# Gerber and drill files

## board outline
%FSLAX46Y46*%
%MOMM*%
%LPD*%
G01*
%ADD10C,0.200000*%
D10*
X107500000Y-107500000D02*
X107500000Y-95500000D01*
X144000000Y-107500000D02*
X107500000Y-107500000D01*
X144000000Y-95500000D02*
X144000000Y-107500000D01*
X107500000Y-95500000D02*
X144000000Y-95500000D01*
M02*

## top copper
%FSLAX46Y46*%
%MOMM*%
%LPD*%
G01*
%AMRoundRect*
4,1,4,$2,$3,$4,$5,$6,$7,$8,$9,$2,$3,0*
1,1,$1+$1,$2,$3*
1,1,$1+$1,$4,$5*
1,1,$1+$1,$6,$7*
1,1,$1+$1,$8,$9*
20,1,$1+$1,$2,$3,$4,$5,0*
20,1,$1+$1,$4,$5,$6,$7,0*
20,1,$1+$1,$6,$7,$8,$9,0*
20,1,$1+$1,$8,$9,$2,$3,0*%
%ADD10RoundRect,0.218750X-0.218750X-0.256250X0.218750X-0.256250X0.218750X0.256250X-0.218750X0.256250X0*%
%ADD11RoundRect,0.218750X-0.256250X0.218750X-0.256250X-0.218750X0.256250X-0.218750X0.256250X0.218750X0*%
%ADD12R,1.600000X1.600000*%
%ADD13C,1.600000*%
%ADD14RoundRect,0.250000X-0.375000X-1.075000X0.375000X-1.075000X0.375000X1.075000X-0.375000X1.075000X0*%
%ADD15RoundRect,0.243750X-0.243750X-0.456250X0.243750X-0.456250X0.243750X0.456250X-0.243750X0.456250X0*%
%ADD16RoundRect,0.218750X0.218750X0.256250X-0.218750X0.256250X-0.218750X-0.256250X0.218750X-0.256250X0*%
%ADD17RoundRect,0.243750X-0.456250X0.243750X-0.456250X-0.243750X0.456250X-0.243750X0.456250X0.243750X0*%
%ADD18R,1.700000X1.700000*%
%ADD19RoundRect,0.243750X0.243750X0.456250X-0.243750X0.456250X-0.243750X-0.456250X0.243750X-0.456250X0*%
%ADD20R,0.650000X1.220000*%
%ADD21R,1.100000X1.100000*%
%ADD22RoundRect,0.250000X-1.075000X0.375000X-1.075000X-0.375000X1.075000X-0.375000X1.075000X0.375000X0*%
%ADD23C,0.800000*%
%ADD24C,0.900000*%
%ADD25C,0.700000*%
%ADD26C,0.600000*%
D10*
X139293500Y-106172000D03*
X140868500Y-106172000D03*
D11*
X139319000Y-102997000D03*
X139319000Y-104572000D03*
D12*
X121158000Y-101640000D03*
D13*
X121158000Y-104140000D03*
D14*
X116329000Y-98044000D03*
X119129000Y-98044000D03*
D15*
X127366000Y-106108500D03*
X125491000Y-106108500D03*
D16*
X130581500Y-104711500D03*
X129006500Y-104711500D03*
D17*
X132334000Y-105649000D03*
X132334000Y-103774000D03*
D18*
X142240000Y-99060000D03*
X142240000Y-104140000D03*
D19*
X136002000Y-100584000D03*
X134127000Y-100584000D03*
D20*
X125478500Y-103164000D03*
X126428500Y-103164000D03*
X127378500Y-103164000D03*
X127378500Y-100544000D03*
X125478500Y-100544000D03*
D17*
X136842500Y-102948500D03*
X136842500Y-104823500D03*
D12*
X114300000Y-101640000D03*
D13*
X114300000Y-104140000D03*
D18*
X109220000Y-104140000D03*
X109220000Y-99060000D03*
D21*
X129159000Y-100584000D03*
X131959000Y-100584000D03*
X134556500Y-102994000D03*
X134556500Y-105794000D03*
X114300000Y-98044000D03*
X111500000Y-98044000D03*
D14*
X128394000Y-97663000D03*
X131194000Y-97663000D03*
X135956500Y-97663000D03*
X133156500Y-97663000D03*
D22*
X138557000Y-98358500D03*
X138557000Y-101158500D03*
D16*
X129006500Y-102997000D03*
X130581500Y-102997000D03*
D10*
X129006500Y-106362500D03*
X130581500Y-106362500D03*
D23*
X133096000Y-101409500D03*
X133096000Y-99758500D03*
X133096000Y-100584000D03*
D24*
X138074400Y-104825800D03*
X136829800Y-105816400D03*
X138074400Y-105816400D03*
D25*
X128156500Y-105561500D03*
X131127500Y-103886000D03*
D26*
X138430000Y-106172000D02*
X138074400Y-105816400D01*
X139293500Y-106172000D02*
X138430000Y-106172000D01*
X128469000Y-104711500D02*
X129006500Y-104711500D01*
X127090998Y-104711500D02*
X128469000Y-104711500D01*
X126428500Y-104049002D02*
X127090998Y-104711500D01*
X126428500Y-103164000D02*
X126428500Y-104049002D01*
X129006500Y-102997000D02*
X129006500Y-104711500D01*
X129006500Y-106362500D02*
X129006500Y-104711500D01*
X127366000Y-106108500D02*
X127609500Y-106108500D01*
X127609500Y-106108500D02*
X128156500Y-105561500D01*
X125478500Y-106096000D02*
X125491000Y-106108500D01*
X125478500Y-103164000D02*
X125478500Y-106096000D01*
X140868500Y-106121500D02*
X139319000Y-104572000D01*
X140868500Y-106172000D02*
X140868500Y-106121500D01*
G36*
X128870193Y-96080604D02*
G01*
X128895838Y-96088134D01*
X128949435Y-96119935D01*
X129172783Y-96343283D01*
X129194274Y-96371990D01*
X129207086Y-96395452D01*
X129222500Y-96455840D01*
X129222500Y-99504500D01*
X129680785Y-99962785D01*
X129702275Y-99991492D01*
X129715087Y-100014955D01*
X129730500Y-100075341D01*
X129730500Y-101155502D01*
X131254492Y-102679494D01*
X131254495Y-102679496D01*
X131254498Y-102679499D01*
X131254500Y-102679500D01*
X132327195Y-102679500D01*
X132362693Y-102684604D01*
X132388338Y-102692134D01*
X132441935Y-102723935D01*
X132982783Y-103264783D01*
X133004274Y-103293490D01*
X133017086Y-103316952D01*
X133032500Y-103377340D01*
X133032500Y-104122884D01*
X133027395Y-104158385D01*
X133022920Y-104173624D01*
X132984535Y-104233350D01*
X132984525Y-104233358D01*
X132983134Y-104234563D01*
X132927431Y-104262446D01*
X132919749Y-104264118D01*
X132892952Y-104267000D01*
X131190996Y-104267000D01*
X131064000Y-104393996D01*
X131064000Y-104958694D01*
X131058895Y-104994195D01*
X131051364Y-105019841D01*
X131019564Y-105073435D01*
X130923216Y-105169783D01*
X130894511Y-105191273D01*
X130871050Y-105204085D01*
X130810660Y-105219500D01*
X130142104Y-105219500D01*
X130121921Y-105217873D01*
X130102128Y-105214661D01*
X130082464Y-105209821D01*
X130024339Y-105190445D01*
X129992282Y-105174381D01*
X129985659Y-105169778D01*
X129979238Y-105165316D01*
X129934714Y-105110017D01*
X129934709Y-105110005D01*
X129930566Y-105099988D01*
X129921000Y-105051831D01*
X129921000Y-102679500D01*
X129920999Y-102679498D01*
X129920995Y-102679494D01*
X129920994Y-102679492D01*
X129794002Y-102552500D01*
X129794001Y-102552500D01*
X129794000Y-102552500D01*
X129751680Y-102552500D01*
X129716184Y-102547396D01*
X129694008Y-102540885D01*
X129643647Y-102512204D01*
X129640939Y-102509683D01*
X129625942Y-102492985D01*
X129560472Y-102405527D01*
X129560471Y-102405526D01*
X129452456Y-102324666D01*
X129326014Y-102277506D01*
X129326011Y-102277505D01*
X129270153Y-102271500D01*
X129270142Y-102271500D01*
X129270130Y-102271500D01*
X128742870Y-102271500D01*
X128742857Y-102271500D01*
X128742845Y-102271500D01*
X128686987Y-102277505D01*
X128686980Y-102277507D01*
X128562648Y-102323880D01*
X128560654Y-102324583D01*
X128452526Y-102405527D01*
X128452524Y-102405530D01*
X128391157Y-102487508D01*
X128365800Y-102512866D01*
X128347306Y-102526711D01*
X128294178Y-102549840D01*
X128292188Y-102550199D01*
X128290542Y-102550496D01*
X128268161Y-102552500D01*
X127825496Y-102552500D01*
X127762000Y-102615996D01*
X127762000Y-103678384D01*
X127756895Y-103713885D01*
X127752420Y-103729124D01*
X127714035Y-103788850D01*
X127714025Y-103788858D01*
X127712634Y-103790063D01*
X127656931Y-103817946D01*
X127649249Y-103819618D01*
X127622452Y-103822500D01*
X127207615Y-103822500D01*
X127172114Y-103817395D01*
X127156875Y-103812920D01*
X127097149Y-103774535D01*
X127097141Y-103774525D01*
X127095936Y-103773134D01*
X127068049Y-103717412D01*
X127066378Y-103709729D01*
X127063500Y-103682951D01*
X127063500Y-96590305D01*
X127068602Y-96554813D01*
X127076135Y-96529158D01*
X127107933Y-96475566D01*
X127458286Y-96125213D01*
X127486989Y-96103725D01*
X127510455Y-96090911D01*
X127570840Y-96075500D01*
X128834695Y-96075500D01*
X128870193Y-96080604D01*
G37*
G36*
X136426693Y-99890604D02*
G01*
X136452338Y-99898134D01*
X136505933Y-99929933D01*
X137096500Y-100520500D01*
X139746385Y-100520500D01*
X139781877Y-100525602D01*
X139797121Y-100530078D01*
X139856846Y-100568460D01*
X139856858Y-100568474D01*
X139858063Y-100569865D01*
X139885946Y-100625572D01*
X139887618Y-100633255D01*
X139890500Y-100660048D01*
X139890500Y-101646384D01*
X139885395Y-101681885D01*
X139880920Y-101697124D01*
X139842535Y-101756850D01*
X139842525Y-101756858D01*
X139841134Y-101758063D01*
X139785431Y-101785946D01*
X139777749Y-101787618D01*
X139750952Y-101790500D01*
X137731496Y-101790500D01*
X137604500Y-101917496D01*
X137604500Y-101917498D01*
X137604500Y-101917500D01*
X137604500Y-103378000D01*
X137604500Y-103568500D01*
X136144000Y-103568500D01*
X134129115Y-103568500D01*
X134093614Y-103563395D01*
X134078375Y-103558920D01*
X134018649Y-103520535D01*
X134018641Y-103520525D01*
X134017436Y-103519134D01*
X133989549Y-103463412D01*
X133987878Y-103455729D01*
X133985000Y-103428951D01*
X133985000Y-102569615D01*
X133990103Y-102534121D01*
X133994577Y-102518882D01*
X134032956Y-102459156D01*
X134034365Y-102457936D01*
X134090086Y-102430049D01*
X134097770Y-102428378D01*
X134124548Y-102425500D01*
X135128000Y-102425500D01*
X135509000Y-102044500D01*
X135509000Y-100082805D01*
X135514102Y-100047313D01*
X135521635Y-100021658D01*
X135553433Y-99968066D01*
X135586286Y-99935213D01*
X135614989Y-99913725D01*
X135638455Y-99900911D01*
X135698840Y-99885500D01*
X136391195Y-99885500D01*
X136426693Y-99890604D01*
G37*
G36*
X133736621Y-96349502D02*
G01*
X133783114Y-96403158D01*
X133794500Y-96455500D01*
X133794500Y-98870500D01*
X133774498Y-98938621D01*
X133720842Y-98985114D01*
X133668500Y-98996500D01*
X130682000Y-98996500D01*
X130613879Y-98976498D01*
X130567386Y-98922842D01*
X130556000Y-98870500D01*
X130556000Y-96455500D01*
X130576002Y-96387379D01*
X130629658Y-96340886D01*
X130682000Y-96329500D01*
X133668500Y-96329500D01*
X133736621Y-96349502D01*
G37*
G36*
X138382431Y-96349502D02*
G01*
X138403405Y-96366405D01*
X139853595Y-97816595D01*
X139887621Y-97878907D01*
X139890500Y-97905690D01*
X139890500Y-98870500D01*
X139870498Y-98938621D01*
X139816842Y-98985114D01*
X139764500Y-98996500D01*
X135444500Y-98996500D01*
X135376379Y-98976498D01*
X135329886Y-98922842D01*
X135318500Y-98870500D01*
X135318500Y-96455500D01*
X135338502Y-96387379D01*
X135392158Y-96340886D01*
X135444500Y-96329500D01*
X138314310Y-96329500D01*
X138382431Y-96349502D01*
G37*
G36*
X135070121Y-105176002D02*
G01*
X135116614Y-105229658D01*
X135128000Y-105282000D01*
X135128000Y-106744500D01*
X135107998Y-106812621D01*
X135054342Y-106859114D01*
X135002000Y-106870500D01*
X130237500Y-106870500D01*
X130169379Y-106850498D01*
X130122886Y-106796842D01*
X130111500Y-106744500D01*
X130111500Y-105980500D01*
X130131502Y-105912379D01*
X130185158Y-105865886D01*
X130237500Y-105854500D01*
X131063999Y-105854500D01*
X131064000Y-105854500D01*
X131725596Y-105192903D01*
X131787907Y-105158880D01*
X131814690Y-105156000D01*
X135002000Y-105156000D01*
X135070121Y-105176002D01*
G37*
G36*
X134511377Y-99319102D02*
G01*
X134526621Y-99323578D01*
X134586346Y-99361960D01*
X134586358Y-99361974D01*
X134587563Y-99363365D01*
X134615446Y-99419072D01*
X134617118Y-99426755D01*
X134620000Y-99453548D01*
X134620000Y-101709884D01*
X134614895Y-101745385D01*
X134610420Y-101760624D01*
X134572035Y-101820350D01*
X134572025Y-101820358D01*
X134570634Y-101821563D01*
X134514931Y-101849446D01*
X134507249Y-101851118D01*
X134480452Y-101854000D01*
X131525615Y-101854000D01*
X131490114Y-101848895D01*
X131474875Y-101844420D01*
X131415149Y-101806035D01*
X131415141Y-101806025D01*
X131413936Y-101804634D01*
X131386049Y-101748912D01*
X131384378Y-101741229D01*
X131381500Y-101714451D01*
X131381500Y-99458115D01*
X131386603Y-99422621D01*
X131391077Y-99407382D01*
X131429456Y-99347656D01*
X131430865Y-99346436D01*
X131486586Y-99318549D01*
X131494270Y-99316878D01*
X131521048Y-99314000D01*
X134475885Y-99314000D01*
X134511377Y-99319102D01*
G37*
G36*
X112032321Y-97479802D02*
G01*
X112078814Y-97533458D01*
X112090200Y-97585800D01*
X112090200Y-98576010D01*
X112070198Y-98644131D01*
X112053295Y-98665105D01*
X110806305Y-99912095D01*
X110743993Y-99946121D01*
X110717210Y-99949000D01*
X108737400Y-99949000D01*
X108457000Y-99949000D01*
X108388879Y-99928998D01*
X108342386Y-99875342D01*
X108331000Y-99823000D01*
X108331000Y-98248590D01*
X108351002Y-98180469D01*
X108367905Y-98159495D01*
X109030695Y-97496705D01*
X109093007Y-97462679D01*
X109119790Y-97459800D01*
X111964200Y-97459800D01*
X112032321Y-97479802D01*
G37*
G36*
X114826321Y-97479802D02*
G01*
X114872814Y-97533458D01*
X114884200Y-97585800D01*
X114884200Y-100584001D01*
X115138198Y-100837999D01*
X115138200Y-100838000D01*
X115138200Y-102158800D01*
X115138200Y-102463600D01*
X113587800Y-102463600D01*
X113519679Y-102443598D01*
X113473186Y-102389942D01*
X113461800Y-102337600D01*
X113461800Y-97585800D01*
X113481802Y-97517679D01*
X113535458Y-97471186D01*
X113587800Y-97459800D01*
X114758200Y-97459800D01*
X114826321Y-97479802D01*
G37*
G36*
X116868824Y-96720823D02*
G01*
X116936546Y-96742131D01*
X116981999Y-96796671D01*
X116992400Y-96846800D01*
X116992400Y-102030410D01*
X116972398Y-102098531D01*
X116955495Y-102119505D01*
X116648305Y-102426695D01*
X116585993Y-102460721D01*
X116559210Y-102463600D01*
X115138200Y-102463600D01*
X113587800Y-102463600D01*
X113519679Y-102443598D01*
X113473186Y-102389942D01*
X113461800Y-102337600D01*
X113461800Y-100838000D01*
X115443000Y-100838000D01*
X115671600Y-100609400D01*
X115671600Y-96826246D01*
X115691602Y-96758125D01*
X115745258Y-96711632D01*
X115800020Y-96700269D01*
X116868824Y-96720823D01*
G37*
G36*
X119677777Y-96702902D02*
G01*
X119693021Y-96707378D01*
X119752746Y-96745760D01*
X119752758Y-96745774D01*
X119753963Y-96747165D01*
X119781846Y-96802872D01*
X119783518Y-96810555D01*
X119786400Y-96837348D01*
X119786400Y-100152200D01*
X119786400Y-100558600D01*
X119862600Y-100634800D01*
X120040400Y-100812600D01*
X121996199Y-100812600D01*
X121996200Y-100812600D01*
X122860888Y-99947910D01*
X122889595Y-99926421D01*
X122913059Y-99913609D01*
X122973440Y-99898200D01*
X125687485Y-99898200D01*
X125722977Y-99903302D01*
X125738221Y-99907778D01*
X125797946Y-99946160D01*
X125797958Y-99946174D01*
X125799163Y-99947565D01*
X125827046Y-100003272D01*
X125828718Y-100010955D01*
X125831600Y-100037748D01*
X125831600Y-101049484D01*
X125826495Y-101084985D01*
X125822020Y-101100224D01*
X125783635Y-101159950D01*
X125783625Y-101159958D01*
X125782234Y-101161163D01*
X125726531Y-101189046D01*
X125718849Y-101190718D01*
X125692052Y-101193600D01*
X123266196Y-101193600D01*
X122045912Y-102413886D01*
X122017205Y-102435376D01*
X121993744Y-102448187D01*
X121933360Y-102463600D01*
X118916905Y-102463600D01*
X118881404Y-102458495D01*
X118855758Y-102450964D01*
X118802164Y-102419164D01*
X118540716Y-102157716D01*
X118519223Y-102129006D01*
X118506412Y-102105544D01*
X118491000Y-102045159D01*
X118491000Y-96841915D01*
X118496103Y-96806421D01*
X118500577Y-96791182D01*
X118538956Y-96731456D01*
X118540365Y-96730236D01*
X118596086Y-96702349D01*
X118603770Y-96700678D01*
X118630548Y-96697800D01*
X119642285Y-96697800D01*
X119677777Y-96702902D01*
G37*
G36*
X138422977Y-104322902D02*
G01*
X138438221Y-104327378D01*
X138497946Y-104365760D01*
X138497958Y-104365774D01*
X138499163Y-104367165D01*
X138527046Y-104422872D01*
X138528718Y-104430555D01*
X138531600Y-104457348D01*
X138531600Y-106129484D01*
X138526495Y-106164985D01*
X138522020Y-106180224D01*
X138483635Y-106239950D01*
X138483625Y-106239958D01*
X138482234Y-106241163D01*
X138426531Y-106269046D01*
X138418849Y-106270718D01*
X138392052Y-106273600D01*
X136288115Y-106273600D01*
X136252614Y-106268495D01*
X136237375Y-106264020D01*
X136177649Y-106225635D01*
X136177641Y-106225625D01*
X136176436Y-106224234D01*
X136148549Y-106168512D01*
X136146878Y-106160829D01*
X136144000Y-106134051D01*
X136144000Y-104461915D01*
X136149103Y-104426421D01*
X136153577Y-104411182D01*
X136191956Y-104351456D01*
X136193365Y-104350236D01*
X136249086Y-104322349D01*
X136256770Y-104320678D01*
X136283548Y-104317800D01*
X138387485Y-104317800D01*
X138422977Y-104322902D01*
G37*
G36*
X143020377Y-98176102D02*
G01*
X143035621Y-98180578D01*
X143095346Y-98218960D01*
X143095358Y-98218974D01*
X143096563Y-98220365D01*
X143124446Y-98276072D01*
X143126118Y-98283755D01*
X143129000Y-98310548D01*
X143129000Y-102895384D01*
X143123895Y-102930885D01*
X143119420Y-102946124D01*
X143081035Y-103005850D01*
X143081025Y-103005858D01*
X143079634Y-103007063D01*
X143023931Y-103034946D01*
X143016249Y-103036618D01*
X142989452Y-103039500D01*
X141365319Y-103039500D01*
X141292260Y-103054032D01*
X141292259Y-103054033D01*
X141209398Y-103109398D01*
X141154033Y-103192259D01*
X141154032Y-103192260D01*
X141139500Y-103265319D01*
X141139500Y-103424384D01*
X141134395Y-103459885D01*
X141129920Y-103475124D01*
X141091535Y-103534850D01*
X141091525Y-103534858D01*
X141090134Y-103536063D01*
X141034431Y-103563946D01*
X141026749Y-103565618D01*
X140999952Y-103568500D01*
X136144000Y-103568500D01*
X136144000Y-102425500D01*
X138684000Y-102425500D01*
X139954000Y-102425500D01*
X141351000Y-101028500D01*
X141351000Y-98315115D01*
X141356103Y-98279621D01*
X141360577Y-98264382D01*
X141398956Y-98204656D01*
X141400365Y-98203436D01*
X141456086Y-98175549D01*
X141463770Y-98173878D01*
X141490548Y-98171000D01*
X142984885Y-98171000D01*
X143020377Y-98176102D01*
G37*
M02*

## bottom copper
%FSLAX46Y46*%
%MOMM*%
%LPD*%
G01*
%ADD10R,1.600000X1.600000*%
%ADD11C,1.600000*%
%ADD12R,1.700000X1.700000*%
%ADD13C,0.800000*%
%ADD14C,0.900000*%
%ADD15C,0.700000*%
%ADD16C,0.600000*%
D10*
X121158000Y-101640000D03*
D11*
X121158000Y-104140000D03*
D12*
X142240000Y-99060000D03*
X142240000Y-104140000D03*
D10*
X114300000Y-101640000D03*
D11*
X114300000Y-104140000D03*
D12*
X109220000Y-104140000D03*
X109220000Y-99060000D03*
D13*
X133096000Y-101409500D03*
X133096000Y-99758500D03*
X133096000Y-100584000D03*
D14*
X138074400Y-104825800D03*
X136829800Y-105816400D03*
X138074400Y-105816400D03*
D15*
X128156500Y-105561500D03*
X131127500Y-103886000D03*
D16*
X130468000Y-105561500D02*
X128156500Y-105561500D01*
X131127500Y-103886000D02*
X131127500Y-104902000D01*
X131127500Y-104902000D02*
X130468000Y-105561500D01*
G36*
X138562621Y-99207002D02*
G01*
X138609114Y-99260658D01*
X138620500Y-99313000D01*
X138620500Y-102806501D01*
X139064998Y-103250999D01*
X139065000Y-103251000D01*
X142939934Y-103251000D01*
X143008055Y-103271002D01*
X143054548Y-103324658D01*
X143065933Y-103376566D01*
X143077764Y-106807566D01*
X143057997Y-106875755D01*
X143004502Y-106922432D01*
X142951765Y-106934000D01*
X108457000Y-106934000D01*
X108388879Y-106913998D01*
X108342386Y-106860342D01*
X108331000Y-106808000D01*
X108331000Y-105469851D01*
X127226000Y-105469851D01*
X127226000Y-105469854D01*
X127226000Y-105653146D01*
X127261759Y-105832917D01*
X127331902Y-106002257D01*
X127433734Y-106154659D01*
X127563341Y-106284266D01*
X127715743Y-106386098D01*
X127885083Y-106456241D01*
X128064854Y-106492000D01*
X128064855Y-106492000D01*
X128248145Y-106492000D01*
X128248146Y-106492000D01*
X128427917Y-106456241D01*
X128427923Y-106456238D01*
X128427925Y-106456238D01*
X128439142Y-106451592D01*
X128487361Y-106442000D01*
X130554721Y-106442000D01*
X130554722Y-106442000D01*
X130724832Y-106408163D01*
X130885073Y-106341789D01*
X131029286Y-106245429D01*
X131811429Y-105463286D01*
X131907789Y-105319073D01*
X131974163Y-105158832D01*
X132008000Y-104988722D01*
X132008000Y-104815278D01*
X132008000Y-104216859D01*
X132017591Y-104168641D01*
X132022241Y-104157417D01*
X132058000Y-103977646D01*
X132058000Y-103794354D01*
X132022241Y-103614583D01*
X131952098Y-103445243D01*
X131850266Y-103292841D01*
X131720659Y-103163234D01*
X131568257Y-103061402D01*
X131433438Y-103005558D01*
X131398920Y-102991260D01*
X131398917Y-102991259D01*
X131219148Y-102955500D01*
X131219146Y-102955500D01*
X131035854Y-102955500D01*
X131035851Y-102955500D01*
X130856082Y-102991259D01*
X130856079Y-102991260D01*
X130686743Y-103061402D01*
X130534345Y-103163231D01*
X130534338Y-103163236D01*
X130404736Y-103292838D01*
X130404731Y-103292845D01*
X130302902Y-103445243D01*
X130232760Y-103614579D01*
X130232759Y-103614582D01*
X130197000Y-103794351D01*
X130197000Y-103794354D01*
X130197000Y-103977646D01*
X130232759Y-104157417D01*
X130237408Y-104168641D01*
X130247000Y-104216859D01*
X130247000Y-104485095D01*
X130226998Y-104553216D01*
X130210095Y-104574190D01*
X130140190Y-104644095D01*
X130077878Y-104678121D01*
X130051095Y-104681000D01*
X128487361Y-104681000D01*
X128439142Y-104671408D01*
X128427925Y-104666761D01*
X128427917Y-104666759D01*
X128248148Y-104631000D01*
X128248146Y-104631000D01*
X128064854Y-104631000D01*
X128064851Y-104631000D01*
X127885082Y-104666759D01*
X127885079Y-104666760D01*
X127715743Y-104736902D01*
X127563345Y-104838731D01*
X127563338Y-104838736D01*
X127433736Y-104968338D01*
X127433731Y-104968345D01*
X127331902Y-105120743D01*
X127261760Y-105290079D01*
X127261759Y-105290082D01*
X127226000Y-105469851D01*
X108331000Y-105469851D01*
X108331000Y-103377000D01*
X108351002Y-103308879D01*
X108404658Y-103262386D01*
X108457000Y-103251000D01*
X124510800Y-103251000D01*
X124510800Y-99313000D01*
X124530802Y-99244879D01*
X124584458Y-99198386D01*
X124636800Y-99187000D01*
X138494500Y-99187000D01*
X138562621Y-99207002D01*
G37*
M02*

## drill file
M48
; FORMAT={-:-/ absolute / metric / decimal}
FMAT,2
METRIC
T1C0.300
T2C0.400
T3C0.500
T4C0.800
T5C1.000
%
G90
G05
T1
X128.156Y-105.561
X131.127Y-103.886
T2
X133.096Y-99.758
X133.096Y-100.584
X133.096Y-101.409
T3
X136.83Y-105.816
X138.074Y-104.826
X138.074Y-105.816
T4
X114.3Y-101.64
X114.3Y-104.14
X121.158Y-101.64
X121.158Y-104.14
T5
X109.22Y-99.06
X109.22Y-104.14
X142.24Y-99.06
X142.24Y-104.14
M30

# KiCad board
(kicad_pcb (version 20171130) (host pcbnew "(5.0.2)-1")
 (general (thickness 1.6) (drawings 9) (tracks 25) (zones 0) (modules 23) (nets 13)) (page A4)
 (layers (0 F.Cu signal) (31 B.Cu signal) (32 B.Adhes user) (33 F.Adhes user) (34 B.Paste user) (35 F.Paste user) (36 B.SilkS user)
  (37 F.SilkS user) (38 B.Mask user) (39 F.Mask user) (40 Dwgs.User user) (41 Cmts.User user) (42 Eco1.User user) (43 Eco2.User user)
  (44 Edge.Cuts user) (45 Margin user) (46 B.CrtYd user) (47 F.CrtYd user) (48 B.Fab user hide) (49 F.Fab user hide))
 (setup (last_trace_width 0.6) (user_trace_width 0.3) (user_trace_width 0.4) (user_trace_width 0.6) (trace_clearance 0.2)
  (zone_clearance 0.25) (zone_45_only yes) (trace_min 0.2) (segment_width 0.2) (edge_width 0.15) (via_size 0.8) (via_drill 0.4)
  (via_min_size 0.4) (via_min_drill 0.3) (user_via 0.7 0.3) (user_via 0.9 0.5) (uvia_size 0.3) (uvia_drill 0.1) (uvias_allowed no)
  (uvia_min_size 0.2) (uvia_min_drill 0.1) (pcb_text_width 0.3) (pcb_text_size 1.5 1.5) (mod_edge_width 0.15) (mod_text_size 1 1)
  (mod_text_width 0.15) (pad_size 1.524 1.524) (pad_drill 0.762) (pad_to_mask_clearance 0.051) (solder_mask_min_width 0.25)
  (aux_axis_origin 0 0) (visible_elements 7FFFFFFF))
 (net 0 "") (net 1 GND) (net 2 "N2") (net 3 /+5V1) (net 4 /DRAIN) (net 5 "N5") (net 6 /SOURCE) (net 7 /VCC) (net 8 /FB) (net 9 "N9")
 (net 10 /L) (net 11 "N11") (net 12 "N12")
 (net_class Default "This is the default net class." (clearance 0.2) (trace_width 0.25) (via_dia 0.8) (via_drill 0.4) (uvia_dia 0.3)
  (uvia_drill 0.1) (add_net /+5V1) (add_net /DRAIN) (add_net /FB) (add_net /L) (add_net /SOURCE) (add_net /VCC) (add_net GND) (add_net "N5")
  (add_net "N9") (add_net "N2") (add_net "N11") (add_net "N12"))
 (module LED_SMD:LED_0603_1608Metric (layer F.Cu) (at 140.081 106.172)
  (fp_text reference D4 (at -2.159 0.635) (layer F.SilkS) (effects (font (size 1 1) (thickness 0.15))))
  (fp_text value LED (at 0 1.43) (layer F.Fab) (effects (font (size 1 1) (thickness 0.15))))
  (pad 1 smd roundrect (at -0.7875 0) (size 0.875 0.95) (layers F.Cu F.Paste F.Mask) (roundrect_rratio 0.25) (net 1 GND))
  (pad 2 smd roundrect (at 0.7875 0) (size 0.875 0.95) (layers F.Cu F.Paste F.Mask) (roundrect_rratio 0.25) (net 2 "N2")))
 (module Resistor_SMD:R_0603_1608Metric (layer F.Cu) (at 139.319 103.7845 270)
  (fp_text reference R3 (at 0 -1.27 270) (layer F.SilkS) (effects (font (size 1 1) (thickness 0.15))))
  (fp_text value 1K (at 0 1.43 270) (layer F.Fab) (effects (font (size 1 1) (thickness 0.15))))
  (pad 1 smd roundrect (at -0.7875 0 270) (size 0.875 0.95) (layers F.Cu F.Paste F.Mask) (roundrect_rratio 0.25) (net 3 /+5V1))
  (pad 2 smd roundrect (at 0.7875 0 270) (size 0.875 0.95) (layers F.Cu F.Paste F.Mask) (roundrect_rratio 0.25) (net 2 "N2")))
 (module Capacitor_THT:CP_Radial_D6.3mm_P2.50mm (layer F.Cu) (at 121.158 101.64 270)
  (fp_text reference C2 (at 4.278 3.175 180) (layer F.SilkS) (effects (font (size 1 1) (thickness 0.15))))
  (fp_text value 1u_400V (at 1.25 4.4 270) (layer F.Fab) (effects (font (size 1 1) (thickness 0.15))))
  (pad 1 thru_hole rect (at 0 0 270) (size 1.6 1.6) (drill 0.8) (layers *.Cu *.Mask) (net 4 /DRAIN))
  (pad 2 thru_hole circle (at 2.5 0 270) (size 1.6 1.6) (drill 0.8) (layers *.Cu *.Mask) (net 1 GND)))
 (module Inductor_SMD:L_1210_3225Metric (layer F.Cu) (at 117.729 98.044)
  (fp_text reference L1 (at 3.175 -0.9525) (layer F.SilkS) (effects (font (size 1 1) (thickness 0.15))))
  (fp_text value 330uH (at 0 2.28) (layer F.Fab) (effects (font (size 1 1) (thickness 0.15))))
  (pad 1 smd roundrect (at -1.4 0) (size 1.25 2.65) (layers F.Cu F.Paste F.Mask) (roundrect_rratio 0.2) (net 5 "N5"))
  (pad 2 smd roundrect (at 1.4 0) (size 1.25 2.65) (layers F.Cu F.Paste F.Mask) (roundrect_rratio 0.2) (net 4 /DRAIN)))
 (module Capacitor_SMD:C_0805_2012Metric (layer F.Cu) (at 126.4285 106.1085)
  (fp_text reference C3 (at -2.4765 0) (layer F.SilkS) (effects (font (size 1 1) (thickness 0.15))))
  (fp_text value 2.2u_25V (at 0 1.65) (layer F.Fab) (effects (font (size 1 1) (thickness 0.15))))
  (pad 2 smd roundrect (at 0.9375 0) (size 0.975 1.4) (layers F.Cu F.Paste F.Mask) (roundrect_rratio 0.25) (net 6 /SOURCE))
  (pad 1 smd roundrect (at -0.9375 0) (size 0.975 1.4) (layers F.Cu F.Paste F.Mask) (roundrect_rratio 0.25) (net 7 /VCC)))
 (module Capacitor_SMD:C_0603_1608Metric (layer F.Cu) (at 129.794 104.7115 180)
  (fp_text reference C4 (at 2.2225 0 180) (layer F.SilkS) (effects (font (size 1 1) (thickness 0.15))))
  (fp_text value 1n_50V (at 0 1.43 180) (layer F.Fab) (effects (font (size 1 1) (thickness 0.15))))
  (pad 1 smd roundrect (at -0.7875 0 180) (size 0.875 0.95) (layers F.Cu F.Paste F.Mask) (roundrect_rratio 0.25) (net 6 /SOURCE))
  (pad 2 smd roundrect (at 0.7875 0 180) (size 0.875 0.95) (layers F.Cu F.Paste F.Mask) (roundrect_rratio 0.25) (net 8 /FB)))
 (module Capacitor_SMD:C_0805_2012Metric (layer F.Cu) (at 132.334 104.7115 270)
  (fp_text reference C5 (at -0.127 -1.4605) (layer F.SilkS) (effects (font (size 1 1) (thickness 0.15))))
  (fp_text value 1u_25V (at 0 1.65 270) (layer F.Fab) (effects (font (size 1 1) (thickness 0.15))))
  (pad 2 smd roundrect (at 0.9375 0 270) (size 0.975 1.4) (layers F.Cu F.Paste F.Mask) (roundrect_rratio 0.25) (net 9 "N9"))
  (pad 1 smd roundrect (at -0.9375 0 270) (size 0.975 1.4) (layers F.Cu F.Paste F.Mask) (roundrect_rratio 0.25) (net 6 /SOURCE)))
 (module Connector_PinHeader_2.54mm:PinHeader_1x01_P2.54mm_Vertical (layer B.Cu) (at 142.24 99.06 180)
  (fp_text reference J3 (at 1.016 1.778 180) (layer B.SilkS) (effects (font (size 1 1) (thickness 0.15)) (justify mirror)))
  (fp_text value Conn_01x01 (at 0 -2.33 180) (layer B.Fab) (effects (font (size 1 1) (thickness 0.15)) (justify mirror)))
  (pad 1 thru_hole rect (at 0 0 180) (size 1.7 1.7) (drill 1) (layers *.Cu *.Mask) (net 3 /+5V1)))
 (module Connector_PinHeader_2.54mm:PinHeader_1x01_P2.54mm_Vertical (layer B.Cu) (at 142.24 104.14 180)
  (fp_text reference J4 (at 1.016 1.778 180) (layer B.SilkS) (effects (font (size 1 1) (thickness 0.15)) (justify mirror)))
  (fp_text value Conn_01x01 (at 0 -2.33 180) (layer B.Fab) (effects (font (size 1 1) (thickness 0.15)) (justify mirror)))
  (pad 1 thru_hole rect (at 0 0 180) (size 1.7 1.7) (drill 1) (layers *.Cu *.Mask) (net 1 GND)))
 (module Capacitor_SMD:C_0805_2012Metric (layer F.Cu) (at 135.0645 100.584 180)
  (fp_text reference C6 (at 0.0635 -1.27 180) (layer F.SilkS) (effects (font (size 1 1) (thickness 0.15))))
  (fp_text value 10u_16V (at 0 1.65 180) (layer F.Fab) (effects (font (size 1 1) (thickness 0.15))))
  (pad 1 smd roundrect (at -0.9375 0 180) (size 0.975 1.4) (layers F.Cu F.Paste F.Mask) (roundrect_rratio 0.25) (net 3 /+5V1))
  (pad 2 smd roundrect (at 0.9375 0 180) (size 0.975 1.4) (layers F.Cu F.Paste F.Mask) (roundrect_rratio 0.25) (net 1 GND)))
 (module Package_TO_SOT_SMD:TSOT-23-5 (layer F.Cu) (at 126.4285 101.854 90)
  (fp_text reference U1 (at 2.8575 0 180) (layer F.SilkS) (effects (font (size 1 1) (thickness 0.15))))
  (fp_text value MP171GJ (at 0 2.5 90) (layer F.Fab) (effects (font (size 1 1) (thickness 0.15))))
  (pad 1 smd rect (at -1.31 -0.95 90) (size 1.22 0.65) (layers F.Cu F.Paste F.Mask) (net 7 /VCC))
  (pad 2 smd rect (at -1.31 0 90) (size 1.22 0.65) (layers F.Cu F.Paste F.Mask) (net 8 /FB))
  (pad 3 smd rect (at -1.31 0.95 90) (size 1.22 0.65) (layers F.Cu F.Paste F.Mask) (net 6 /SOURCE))
  (pad 4 smd rect (at 1.31 0.95 90) (size 1.22 0.65) (layers F.Cu F.Paste F.Mask) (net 6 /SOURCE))
  (pad 5 smd rect (at 1.31 -0.95 90) (size 1.22 0.65) (layers F.Cu F.Paste F.Mask) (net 4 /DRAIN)))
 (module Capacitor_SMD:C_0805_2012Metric (layer F.Cu) (at 136.8425 103.886 270)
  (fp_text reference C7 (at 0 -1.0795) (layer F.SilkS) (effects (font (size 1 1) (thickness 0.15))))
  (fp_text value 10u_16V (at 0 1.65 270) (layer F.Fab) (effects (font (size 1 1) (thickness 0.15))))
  (pad 1 smd roundrect (at -0.9375 0 270) (size 0.975 1.4) (layers F.Cu F.Paste F.Mask) (roundrect_rratio 0.25) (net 3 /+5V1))
  (pad 2 smd roundrect (at 0.9375 0 270) (size 0.975 1.4) (layers F.Cu F.Paste F.Mask) (roundrect_rratio 0.25) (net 1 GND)))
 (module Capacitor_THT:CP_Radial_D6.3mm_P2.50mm (layer F.Cu) (at 114.3 101.64 270)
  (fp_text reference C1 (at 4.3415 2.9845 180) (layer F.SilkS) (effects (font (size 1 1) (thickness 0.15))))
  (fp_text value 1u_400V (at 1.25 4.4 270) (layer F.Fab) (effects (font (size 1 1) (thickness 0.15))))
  (pad 1 thru_hole rect (at 0 0 270) (size 1.6 1.6) (drill 0.8) (layers *.Cu *.Mask) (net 5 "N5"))
  (pad 2 thru_hole circle (at 2.5 0 270) (size 1.6 1.6) (drill 0.8) (layers *.Cu *.Mask) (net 1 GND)))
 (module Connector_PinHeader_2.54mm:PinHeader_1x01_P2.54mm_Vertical (layer B.Cu) (at 109.22 104.14)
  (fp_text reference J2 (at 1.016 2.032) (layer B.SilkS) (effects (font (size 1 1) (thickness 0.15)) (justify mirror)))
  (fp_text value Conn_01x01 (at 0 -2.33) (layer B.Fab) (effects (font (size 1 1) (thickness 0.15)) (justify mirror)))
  (pad 1 thru_hole rect (at 0 0) (size 1.7 1.7) (drill 1) (layers *.Cu *.Mask) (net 1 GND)))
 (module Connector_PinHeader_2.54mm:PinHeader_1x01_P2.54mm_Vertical (layer B.Cu) (at 109.22 99.06)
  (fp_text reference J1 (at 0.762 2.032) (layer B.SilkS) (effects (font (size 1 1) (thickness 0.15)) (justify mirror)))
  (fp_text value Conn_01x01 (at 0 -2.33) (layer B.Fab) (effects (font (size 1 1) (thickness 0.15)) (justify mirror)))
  (pad 1 thru_hole rect (at 0 0) (size 1.7 1.7) (drill 1) (layers *.Cu *.Mask) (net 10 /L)))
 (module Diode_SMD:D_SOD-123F (layer F.Cu) (at 130.559 100.584)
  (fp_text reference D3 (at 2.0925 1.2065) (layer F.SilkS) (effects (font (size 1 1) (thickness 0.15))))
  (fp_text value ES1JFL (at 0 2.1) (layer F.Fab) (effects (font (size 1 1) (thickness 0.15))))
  (pad 1 smd rect (at -1.4 0) (size 1.1 1.1) (layers F.Cu F.Paste F.Mask) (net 6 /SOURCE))
  (pad 2 smd rect (at 1.4 0) (size 1.1 1.1) (layers F.Cu F.Paste F.Mask) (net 1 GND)))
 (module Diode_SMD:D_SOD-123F (layer F.Cu) (at 134.5565 104.394 90)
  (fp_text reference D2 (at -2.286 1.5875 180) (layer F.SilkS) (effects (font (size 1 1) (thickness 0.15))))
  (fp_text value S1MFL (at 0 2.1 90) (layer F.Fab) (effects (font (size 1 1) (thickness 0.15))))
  (pad 2 smd rect (at 1.4 0 90) (size 1.1 1.1) (layers F.Cu F.Paste F.Mask) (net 3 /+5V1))
  (pad 1 smd rect (at -1.4 0 90) (size 1.1 1.1) (layers F.Cu F.Paste F.Mask) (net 9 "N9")))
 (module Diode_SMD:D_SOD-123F (layer F.Cu) (at 112.9 98.044 180)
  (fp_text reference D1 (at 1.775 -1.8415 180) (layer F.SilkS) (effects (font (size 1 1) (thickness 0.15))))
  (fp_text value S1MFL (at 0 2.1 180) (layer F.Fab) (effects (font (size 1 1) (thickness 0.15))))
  (pad 1 smd rect (at -1.4 0 180) (size 1.1 1.1) (layers F.Cu F.Paste F.Mask) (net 5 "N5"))
  (pad 2 smd rect (at 1.4 0 180) (size 1.1 1.1) (layers F.Cu F.Paste F.Mask) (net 10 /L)))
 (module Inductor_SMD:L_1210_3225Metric (layer F.Cu) (at 129.794 97.663)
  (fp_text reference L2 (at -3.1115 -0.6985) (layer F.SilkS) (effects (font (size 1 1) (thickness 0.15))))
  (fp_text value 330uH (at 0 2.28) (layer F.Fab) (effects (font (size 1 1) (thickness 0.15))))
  (pad 1 smd roundrect (at -1.4 0) (size 1.25 2.65) (layers F.Cu F.Paste F.Mask) (roundrect_rratio 0.2) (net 6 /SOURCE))
  (pad 2 smd roundrect (at 1.4 0) (size 1.25 2.65) (layers F.Cu F.Paste F.Mask) (roundrect_rratio 0.2) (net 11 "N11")))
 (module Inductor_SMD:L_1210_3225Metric (layer F.Cu) (at 134.5565 97.663)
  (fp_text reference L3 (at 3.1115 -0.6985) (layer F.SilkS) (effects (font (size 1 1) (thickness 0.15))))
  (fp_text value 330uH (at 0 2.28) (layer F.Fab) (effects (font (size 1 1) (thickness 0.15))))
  (pad 2 smd roundrect (at 1.4 0) (size 1.25 2.65) (layers F.Cu F.Paste F.Mask) (roundrect_rratio 0.2) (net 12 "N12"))
  (pad 1 smd roundrect (at -1.4 0) (size 1.25 2.65) (layers F.Cu F.Paste F.Mask) (roundrect_rratio 0.2) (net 11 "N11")))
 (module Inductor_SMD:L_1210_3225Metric (layer F.Cu) (at 138.557 99.7585 270)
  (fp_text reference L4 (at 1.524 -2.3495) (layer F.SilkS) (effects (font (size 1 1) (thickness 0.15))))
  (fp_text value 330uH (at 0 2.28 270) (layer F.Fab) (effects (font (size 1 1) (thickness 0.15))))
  (pad 1 smd roundrect (at -1.4 0 270) (size 1.25 2.65) (layers F.Cu F.Paste F.Mask) (roundrect_rratio 0.2) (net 12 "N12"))
  (pad 2 smd roundrect (at 1.4 0 270) (size 1.25 2.65) (layers F.Cu F.Paste F.Mask) (roundrect_rratio 0.2) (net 3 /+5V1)))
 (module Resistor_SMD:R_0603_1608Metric (layer F.Cu) (at 129.794 102.997 180)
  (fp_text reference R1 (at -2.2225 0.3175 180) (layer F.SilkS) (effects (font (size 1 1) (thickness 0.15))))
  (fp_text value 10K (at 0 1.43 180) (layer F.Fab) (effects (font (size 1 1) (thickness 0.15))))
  (pad 2 smd roundrect (at 0.7875 0 180) (size 0.875 0.95) (layers F.Cu F.Paste F.Mask) (roundrect_rratio 0.25) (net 8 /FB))
  (pad 1 smd roundrect (at -0.7875 0 180) (size 0.875 0.95) (layers F.Cu F.Paste F.Mask) (roundrect_rratio 0.25) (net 6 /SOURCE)))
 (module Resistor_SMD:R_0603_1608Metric (layer F.Cu) (at 129.794 106.3625)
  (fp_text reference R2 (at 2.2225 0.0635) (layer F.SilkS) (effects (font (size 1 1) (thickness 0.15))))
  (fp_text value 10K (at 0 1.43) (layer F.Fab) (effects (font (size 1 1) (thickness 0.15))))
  (pad 1 smd roundrect (at -0.7875 0) (size 0.875 0.95) (layers F.Cu F.Paste F.Mask) (roundrect_rratio 0.25) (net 8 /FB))
  (pad 2 smd roundrect (at 0.7875 0) (size 0.875 0.95) (layers F.Cu F.Paste F.Mask) (roundrect_rratio 0.25) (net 9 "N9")))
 (gr_line (start 107.5 107.5) (end 107.5 95.5) (layer Edge.Cuts) (width 0.2))
 (gr_line (start 144 107.5) (end 107.5 107.5) (layer Edge.Cuts) (width 0.2))
 (gr_line (start 144 95.5) (end 144 107.5) (layer Edge.Cuts) (width 0.2))
 (gr_line (start 107.5 95.5) (end 144 95.5) (layer Edge.Cuts) (width 0.2))
 (via (at 133.096 101.4095) (size 0.8) (drill 0.4) (layers F.Cu B.Cu) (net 1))
 (via (at 133.096 99.7585) (size 0.8) (drill 0.4) (layers F.Cu B.Cu) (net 1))
 (via (at 133.096 100.584) (size 0.8) (drill 0.4) (layers F.Cu B.Cu) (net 1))
 (via (at 138.0744 104.8258) (size 0.9) (drill 0.5) (layers F.Cu B.Cu) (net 1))
 (via (at 136.8298 105.8164) (size 0.9) (drill 0.5) (layers F.Cu B.Cu) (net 1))
 (via (at 138.0744 105.8164) (size 0.9) (drill 0.5) (layers F.Cu B.Cu) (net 1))
 (segment (start 138.43 106.172) (end 138.0744 105.8164) (width 0.6) (layer F.Cu) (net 1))
 (segment (start 139.2935 106.172) (end 138.43 106.172) (width 0.6) (layer F.Cu) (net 1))
 (segment (start 128.469 104.7115) (end 129.0065 104.7115) (width 0.6) (layer F.Cu) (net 8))
 (segment (start 127.090998 104.7115) (end 128.469 104.7115) (width 0.6) (layer F.Cu) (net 8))
 (segment (start 126.4285 104.049002) (end 127.090998 104.7115) (width 0.6) (layer F.Cu) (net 8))
 (segment (start 126.4285 103.164) (end 126.4285 104.049002) (width 0.6) (layer F.Cu) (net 8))
 (segment (start 129.0065 102.997) (end 129.0065 104.7115) (width 0.6) (layer F.Cu) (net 8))
 (segment (start 129.0065 106.3625) (end 129.0065 104.7115) (width 0.6) (layer F.Cu) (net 8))
 (via (at 128.1565 105.5615) (size 0.7) (drill 0.3) (layers F.Cu B.Cu) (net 6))
 (segment (start 127.366 106.1085) (end 127.6095 106.1085) (width 0.6) (layer F.Cu) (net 6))
 (segment (start 127.6095 106.1085) (end 128.1565 105.5615) (width 0.6) (layer F.Cu) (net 6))
 (via (at 131.1275 103.886) (size 0.7) (drill 0.3) (layers F.Cu B.Cu) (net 6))
 (segment (start 130.468 105.5615) (end 128.1565 105.5615) (width 0.6) (layer B.Cu) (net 6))
 (segment (start 131.1275 103.886) (end 131.1275 104.902) (width 0.6) (layer B.Cu) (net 6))
 (segment (start 131.1275 104.902) (end 130.468 105.5615) (width 0.6) (layer B.Cu) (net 6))
 (segment (start 125.4785 106.096) (end 125.491 106.1085) (width 0.6) (layer F.Cu) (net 7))
 (segment (start 125.4785 103.164) (end 125.4785 106.096) (width 0.6) (layer F.Cu) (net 7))
 (segment (start 140.8685 106.1215) (end 139.319 104.572) (width 0.6) (layer F.Cu) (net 2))
 (segment (start 140.8685 106.172) (end 140.8685 106.1215) (width 0.6) (layer F.Cu) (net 2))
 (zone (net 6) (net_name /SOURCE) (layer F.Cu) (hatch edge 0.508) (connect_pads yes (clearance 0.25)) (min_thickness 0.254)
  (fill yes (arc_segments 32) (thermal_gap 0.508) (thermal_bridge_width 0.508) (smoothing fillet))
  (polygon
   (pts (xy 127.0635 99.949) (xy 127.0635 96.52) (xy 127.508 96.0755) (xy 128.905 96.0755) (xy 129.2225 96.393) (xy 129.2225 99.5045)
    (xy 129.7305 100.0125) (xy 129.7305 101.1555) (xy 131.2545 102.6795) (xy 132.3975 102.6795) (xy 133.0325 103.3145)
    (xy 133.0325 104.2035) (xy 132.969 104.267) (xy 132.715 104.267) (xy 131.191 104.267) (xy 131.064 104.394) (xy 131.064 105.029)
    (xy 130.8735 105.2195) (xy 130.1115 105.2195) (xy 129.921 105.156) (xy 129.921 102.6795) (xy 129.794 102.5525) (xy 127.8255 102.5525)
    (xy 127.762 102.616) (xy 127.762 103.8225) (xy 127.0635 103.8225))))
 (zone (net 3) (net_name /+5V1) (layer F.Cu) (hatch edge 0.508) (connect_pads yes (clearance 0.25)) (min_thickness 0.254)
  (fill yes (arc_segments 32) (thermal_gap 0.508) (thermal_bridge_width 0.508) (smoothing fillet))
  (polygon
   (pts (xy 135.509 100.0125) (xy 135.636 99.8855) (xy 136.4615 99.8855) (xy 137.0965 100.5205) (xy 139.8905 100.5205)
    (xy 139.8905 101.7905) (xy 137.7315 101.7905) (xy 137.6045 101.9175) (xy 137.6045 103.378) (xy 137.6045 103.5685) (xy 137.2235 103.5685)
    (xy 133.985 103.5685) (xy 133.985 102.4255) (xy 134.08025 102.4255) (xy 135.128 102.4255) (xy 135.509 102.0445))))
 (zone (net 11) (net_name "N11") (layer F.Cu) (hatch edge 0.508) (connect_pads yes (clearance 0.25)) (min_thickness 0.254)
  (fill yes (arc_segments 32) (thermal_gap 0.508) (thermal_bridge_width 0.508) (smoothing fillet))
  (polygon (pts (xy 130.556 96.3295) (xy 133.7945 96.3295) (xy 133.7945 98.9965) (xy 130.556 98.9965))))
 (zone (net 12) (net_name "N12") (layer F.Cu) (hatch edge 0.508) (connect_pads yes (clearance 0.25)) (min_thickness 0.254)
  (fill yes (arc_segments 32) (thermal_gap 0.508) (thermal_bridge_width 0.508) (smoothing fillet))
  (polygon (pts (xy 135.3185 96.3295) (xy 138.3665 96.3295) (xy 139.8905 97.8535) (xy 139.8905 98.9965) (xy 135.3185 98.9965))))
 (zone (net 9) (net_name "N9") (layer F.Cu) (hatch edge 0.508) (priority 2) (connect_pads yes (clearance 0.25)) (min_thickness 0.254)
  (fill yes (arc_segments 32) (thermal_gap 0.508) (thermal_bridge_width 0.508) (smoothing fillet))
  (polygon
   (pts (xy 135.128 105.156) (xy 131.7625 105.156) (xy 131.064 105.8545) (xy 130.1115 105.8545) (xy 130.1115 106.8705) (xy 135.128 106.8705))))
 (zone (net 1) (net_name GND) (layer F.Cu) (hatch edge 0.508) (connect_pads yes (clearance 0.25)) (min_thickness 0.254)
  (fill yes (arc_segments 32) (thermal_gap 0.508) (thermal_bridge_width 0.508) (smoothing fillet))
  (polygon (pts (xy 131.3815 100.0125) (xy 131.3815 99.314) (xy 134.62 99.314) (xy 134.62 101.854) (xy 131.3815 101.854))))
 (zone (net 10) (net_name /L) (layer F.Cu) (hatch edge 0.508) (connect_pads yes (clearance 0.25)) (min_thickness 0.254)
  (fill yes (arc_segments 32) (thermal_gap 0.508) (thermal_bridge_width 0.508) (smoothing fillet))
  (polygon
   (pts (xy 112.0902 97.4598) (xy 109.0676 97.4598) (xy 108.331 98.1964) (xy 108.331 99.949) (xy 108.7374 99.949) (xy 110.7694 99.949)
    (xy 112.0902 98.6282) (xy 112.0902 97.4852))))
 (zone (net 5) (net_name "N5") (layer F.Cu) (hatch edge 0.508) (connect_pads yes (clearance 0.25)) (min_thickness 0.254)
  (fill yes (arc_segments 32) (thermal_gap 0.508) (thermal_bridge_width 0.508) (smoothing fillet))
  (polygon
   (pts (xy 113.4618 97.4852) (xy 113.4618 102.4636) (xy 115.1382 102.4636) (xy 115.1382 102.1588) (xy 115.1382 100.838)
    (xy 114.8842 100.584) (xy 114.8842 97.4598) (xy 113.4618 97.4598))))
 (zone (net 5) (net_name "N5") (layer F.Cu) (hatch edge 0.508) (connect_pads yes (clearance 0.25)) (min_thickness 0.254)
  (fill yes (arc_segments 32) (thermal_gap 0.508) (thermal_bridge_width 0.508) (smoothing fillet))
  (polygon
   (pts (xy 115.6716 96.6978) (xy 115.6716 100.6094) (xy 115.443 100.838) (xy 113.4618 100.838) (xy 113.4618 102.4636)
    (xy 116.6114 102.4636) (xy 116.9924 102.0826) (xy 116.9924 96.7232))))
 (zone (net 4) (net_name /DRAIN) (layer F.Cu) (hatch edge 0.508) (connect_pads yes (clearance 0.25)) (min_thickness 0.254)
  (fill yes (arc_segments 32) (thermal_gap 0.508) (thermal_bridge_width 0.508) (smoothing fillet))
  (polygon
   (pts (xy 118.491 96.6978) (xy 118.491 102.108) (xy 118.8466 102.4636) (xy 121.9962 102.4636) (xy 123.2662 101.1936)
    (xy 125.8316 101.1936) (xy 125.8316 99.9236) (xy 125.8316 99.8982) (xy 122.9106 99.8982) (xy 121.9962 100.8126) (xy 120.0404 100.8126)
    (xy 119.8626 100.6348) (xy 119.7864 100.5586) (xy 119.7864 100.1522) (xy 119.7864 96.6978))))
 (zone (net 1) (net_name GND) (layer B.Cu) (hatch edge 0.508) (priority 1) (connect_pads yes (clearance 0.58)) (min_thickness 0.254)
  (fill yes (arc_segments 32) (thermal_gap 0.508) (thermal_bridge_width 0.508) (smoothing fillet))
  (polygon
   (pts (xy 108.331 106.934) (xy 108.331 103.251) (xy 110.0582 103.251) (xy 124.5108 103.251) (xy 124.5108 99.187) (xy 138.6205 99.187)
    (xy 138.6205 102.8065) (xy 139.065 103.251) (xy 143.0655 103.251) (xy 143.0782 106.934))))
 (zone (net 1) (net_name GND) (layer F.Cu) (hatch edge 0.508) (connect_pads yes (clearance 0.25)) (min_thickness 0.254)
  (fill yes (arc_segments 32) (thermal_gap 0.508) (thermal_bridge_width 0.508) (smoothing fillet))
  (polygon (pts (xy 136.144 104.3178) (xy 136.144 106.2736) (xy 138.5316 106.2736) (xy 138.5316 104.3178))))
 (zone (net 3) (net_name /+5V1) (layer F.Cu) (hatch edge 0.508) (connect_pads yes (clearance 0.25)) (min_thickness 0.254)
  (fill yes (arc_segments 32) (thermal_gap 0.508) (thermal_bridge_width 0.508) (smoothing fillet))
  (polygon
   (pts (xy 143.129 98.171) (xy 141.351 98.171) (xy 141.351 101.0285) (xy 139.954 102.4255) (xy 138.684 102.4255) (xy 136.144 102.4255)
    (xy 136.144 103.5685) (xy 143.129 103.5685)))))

